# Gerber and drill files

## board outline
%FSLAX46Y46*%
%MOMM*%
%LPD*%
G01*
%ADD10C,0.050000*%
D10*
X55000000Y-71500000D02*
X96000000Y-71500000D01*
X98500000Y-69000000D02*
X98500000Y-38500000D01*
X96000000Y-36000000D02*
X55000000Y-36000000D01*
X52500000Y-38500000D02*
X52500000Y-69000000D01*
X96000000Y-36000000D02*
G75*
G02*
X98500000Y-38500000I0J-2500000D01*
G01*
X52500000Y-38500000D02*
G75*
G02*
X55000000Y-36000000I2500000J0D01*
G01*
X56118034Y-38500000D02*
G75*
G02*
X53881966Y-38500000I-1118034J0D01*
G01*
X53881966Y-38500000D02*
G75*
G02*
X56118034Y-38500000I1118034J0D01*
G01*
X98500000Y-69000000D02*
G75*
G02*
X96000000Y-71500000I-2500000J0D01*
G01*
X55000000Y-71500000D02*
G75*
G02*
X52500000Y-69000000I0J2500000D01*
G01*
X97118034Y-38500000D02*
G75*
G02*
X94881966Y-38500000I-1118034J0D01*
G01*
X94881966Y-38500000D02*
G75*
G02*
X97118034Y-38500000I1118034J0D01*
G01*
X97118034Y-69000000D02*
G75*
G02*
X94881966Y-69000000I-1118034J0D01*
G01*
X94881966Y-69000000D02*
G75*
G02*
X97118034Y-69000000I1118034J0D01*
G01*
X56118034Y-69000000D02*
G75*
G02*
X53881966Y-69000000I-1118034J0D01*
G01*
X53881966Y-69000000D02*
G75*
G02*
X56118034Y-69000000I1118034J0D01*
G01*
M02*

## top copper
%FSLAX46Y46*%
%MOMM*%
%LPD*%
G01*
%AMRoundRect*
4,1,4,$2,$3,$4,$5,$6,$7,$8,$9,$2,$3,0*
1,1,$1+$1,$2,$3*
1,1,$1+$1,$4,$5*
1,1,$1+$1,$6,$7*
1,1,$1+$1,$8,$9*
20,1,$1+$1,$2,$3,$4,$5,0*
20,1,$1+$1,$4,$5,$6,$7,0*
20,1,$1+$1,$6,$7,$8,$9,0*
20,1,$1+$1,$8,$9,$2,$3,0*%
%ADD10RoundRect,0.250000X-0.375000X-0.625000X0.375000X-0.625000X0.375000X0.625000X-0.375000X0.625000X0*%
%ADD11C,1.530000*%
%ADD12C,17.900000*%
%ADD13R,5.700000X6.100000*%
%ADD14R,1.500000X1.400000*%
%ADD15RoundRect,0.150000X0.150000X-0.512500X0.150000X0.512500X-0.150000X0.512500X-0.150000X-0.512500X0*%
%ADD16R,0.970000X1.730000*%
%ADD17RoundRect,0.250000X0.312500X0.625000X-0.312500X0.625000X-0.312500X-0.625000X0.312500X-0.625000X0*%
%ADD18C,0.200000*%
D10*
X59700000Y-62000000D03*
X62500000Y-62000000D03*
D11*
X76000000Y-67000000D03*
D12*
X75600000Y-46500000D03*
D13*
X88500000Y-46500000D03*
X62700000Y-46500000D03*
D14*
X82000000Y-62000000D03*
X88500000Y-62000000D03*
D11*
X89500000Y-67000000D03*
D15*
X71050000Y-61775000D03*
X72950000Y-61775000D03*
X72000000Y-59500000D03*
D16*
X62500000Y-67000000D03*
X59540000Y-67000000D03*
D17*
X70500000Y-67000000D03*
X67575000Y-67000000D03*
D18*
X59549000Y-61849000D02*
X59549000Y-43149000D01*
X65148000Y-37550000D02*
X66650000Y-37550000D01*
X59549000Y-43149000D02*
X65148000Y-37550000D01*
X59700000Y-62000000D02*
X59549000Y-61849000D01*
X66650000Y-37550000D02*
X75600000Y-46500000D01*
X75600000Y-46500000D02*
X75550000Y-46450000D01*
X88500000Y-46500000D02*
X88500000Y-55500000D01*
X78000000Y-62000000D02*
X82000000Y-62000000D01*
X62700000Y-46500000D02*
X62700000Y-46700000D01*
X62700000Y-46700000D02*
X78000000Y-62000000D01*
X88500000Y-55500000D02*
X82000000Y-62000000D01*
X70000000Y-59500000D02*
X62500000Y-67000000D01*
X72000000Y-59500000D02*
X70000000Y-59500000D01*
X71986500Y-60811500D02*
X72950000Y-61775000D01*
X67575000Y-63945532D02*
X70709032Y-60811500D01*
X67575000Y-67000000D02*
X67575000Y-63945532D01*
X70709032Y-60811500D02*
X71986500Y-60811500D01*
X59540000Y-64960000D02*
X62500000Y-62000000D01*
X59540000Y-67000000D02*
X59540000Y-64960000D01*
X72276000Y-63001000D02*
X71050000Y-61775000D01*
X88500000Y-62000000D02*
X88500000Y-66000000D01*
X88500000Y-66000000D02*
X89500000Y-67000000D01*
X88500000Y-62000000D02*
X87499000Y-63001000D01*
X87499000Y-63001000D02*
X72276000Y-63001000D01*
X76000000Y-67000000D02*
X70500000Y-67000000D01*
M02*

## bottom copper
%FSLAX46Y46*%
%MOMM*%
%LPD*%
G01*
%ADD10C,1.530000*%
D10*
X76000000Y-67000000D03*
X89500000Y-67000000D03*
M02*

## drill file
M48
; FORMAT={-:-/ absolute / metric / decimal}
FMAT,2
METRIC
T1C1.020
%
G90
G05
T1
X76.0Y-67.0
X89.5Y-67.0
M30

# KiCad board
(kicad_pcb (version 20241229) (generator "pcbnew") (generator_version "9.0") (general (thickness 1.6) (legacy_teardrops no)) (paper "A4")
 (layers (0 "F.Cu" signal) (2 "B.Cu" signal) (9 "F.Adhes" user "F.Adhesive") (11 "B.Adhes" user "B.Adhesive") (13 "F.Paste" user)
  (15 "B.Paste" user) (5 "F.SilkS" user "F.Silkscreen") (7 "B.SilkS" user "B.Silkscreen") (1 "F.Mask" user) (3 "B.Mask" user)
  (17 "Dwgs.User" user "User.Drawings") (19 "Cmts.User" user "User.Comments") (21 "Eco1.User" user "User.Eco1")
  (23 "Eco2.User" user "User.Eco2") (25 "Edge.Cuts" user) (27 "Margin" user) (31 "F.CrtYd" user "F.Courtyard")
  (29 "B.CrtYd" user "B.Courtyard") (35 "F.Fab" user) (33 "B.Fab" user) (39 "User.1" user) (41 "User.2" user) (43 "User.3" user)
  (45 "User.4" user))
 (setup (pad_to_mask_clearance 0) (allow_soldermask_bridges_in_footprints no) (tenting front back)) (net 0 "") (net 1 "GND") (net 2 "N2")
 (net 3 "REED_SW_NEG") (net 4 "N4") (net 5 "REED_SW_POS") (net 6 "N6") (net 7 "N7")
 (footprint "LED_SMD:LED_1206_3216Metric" (layer "F.Cu") (at 61.1 62)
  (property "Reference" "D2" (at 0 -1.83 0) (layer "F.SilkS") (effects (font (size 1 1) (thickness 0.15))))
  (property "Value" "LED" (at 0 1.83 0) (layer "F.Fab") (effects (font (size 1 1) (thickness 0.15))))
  (pad "1" smd roundrect (at -1.4 0) (size 1.25 1.75) (layers "F.Cu" "F.Mask" "F.Paste") (roundrect_rratio 0.2) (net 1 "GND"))
  (pad "2" smd roundrect (at 1.4 0) (size 1.25 1.75) (layers "F.Cu" "F.Mask" "F.Paste") (roundrect_rratio 0.2) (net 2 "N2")))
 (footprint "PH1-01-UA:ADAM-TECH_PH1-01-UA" (layer "F.Cu") (at 76 67)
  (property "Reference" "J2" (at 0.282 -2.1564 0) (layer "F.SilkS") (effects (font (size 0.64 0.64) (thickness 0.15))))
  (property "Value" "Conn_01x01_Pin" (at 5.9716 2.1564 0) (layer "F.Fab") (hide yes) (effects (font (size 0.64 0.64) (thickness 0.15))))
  (pad "1" thru_hole circle (at 0 0) (size 1.53 1.53) (drill 1.02) (layers "*.Cu" "*.Mask") (remove_unused_layers no) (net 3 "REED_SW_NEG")
   (solder_mask_margin 0.102)))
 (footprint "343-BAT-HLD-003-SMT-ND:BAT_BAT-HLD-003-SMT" (layer "F.Cu") (at 75.6 46.5 180)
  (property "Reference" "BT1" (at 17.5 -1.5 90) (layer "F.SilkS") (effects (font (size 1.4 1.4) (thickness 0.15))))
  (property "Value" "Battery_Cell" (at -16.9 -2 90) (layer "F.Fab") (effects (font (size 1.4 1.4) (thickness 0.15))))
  (pad "N" smd circle (at 0 0 180) (size 17.9 17.9) (layers "F.Cu" "F.Mask") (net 1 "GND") (solder_mask_margin 0.102))
  (pad "P1" smd rect (at -12.9 0 180) (size 5.7 6.1) (layers "F.Cu" "F.Mask" "F.Paste") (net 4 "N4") (solder_mask_margin 0.102))
  (pad "P1" smd rect (at 12.9 0 180) (size 5.7 6.1) (layers "F.Cu" "F.Mask" "F.Paste") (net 4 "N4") (solder_mask_margin 0.102)))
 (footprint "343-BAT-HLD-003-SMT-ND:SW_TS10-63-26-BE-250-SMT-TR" (layer "F.Cu") (at 85.25 62)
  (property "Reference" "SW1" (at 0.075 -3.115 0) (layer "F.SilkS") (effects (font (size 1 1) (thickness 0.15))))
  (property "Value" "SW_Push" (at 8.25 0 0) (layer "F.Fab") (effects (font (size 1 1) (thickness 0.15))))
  (pad "1" smd rect (at -3.25 0) (size 1.5 1.4) (layers "F.Cu" "F.Mask" "F.Paste") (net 4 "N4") (solder_mask_margin 0.102))
  (pad "2" smd rect (at 3.25 0) (size 1.5 1.4) (layers "F.Cu" "F.Mask" "F.Paste") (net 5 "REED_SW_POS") (solder_mask_margin 0.102)))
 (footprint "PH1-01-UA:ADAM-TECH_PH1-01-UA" (layer "F.Cu") (at 89.5 67)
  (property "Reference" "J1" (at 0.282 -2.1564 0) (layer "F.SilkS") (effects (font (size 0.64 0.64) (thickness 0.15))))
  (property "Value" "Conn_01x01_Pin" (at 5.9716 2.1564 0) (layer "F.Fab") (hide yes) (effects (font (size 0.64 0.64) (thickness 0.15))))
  (pad "1" thru_hole circle (at 0 0) (size 1.53 1.53) (drill 1.02) (layers "*.Cu" "*.Mask") (remove_unused_layers no) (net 5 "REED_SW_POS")
   (solder_mask_margin 0.102)))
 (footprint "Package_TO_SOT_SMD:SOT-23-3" (layer "F.Cu") (at 72 60.6375 90)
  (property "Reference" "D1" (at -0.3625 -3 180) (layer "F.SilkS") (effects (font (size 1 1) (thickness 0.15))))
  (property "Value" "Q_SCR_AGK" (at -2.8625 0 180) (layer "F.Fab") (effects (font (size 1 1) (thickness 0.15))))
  (pad "1" smd roundrect (at -1.1375 -0.95 90) (size 1.325 0.6) (layers "F.Cu" "F.Mask" "F.Paste") (roundrect_rratio 0.25)
   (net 5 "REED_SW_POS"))
  (pad "2" smd roundrect (at -1.1375 0.95 90) (size 1.325 0.6) (layers "F.Cu" "F.Mask" "F.Paste") (roundrect_rratio 0.25) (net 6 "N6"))
  (pad "3" smd roundrect (at 1.1375 0 90) (size 1.325 0.6) (layers "F.Cu" "F.Mask" "F.Paste") (roundrect_rratio 0.25) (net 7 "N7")))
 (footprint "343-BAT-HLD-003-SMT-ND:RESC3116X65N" (layer "F.Cu") (at 61.02 67 180)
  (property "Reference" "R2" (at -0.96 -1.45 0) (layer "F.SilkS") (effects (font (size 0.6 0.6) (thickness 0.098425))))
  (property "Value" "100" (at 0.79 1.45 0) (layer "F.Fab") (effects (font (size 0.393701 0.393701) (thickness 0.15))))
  (pad "1" smd rect (at -1.48 0 180) (size 0.97 1.73) (layers "F.Cu" "F.Mask" "F.Paste") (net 7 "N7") (solder_mask_margin 0.102))
  (pad "2" smd rect (at 1.48 0 180) (size 0.97 1.73) (layers "F.Cu" "F.Mask" "F.Paste") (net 2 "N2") (solder_mask_margin 0.102)))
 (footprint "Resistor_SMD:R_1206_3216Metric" (layer "F.Cu") (at 69.0375 67 180)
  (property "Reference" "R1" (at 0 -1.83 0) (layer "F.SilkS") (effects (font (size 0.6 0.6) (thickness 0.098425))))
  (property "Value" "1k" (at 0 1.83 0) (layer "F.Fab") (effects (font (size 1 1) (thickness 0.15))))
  (pad "1" smd roundrect (at -1.4625 0 180) (size 1.125 1.75) (layers "F.Cu" "F.Mask" "F.Paste") (roundrect_rratio 0.222222)
   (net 3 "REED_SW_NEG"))
  (pad "2" smd roundrect (at 1.4625 0 180) (size 1.125 1.75) (layers "F.Cu" "F.Mask" "F.Paste") (roundrect_rratio 0.222222) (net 6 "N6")))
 (gr_line (start 55 71.5) (end 96 71.5) (stroke (width 0.05) (type default)) (layer "Edge.Cuts"))
 (gr_line (start 98.5 69) (end 98.5 38.5) (stroke (width 0.05) (type default)) (layer "Edge.Cuts"))
 (gr_line (start 96 36) (end 55 36) (stroke (width 0.05) (type default)) (layer "Edge.Cuts"))
 (gr_line (start 52.5 38.5) (end 52.5 69) (stroke (width 0.05) (type default)) (layer "Edge.Cuts"))
 (gr_arc (start 96 36) (mid 97.767767 36.732233) (end 98.5 38.5) (stroke (width 0.05) (type default)) (layer "Edge.Cuts"))
 (gr_arc (start 52.5 38.5) (mid 53.232233 36.732233) (end 55 36) (stroke (width 0.05) (type default)) (layer "Edge.Cuts"))
 (gr_circle (center 55 38.5) (end 56 39) (stroke (width 0.05) (type default)) (fill no) (layer "Edge.Cuts"))
 (gr_arc (start 98.5 69) (mid 97.767767 70.767767) (end 96 71.5) (stroke (width 0.05) (type default)) (layer "Edge.Cuts"))
 (gr_arc (start 55 71.5) (mid 53.232233 70.767767) (end 52.5 69) (stroke (width 0.05) (type default)) (layer "Edge.Cuts"))
 (gr_circle (center 96 38.5) (end 97 38) (stroke (width 0.05) (type default)) (fill no) (layer "Edge.Cuts"))
 (gr_circle (center 96 69) (end 97 69.5) (stroke (width 0.05) (type default)) (fill no) (layer "Edge.Cuts"))
 (gr_circle (center 55 69) (end 56 69.5) (stroke (width 0.05) (type default)) (fill no) (layer "Edge.Cuts"))
 (segment (start 59.549 61.849) (end 59.549 43.149) (width 0.2) (layer "F.Cu") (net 1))
 (segment (start 65.148 37.55) (end 66.65 37.55) (width 0.2) (layer "F.Cu") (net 1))
 (segment (start 59.549 43.149) (end 65.148 37.55) (width 0.2) (layer "F.Cu") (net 1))
 (segment (start 59.7 62) (end 59.549 61.849) (width 0.2) (layer "F.Cu") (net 1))
 (segment (start 66.65 37.55) (end 75.6 46.5) (width 0.2) (layer "F.Cu") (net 1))
 (segment (start 75.6 46.5) (end 75.55 46.45) (width 0.2) (layer "F.Cu") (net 1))
 (segment (start 88.5 46.5) (end 88.5 55.5) (width 0.2) (layer "F.Cu") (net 4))
 (segment (start 78 62) (end 82 62) (width 0.2) (layer "F.Cu") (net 4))
 (segment (start 62.7 46.5) (end 62.7 46.7) (width 0.2) (layer "F.Cu") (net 4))
 (segment (start 62.7 46.7) (end 78 62) (width 0.2) (layer "F.Cu") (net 4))
 (segment (start 88.5 55.5) (end 82 62) (width 0.2) (layer "F.Cu") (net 4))
 (segment (start 70 59.5) (end 62.5 67) (width 0.2) (layer "F.Cu") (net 7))
 (segment (start 72 59.5) (end 70 59.5) (width 0.2) (layer "F.Cu") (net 7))
 (segment (start 71.9865 60.8115) (end 72.95 61.775) (width 0.2) (layer "F.Cu") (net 6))
 (segment (start 67.575 63.945532) (end 70.709032 60.8115) (width 0.2) (layer "F.Cu") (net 6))
 (segment (start 67.575 67) (end 67.575 63.945532) (width 0.2) (layer "F.Cu") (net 6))
 (segment (start 70.709032 60.8115) (end 71.9865 60.8115) (width 0.2) (layer "F.Cu") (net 6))
 (segment (start 59.54 64.96) (end 62.5 62) (width 0.2) (layer "F.Cu") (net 2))
 (segment (start 59.54 67) (end 59.54 64.96) (width 0.2) (layer "F.Cu") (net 2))
 (segment (start 72.276 63.001) (end 71.05 61.775) (width 0.2) (layer "F.Cu") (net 5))
 (segment (start 88.5 62) (end 88.5 66) (width 0.2) (layer "F.Cu") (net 5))
 (segment (start 88.5 66) (end 89.5 67) (width 0.2) (layer "F.Cu") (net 5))
 (segment (start 88.5 62) (end 87.499 63.001) (width 0.2) (layer "F.Cu") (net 5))
 (segment (start 87.499 63.001) (end 72.276 63.001) (width 0.2) (layer "F.Cu") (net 5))
 (segment (start 76 67) (end 70.5 67) (width 0.2) (layer "F.Cu") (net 3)))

